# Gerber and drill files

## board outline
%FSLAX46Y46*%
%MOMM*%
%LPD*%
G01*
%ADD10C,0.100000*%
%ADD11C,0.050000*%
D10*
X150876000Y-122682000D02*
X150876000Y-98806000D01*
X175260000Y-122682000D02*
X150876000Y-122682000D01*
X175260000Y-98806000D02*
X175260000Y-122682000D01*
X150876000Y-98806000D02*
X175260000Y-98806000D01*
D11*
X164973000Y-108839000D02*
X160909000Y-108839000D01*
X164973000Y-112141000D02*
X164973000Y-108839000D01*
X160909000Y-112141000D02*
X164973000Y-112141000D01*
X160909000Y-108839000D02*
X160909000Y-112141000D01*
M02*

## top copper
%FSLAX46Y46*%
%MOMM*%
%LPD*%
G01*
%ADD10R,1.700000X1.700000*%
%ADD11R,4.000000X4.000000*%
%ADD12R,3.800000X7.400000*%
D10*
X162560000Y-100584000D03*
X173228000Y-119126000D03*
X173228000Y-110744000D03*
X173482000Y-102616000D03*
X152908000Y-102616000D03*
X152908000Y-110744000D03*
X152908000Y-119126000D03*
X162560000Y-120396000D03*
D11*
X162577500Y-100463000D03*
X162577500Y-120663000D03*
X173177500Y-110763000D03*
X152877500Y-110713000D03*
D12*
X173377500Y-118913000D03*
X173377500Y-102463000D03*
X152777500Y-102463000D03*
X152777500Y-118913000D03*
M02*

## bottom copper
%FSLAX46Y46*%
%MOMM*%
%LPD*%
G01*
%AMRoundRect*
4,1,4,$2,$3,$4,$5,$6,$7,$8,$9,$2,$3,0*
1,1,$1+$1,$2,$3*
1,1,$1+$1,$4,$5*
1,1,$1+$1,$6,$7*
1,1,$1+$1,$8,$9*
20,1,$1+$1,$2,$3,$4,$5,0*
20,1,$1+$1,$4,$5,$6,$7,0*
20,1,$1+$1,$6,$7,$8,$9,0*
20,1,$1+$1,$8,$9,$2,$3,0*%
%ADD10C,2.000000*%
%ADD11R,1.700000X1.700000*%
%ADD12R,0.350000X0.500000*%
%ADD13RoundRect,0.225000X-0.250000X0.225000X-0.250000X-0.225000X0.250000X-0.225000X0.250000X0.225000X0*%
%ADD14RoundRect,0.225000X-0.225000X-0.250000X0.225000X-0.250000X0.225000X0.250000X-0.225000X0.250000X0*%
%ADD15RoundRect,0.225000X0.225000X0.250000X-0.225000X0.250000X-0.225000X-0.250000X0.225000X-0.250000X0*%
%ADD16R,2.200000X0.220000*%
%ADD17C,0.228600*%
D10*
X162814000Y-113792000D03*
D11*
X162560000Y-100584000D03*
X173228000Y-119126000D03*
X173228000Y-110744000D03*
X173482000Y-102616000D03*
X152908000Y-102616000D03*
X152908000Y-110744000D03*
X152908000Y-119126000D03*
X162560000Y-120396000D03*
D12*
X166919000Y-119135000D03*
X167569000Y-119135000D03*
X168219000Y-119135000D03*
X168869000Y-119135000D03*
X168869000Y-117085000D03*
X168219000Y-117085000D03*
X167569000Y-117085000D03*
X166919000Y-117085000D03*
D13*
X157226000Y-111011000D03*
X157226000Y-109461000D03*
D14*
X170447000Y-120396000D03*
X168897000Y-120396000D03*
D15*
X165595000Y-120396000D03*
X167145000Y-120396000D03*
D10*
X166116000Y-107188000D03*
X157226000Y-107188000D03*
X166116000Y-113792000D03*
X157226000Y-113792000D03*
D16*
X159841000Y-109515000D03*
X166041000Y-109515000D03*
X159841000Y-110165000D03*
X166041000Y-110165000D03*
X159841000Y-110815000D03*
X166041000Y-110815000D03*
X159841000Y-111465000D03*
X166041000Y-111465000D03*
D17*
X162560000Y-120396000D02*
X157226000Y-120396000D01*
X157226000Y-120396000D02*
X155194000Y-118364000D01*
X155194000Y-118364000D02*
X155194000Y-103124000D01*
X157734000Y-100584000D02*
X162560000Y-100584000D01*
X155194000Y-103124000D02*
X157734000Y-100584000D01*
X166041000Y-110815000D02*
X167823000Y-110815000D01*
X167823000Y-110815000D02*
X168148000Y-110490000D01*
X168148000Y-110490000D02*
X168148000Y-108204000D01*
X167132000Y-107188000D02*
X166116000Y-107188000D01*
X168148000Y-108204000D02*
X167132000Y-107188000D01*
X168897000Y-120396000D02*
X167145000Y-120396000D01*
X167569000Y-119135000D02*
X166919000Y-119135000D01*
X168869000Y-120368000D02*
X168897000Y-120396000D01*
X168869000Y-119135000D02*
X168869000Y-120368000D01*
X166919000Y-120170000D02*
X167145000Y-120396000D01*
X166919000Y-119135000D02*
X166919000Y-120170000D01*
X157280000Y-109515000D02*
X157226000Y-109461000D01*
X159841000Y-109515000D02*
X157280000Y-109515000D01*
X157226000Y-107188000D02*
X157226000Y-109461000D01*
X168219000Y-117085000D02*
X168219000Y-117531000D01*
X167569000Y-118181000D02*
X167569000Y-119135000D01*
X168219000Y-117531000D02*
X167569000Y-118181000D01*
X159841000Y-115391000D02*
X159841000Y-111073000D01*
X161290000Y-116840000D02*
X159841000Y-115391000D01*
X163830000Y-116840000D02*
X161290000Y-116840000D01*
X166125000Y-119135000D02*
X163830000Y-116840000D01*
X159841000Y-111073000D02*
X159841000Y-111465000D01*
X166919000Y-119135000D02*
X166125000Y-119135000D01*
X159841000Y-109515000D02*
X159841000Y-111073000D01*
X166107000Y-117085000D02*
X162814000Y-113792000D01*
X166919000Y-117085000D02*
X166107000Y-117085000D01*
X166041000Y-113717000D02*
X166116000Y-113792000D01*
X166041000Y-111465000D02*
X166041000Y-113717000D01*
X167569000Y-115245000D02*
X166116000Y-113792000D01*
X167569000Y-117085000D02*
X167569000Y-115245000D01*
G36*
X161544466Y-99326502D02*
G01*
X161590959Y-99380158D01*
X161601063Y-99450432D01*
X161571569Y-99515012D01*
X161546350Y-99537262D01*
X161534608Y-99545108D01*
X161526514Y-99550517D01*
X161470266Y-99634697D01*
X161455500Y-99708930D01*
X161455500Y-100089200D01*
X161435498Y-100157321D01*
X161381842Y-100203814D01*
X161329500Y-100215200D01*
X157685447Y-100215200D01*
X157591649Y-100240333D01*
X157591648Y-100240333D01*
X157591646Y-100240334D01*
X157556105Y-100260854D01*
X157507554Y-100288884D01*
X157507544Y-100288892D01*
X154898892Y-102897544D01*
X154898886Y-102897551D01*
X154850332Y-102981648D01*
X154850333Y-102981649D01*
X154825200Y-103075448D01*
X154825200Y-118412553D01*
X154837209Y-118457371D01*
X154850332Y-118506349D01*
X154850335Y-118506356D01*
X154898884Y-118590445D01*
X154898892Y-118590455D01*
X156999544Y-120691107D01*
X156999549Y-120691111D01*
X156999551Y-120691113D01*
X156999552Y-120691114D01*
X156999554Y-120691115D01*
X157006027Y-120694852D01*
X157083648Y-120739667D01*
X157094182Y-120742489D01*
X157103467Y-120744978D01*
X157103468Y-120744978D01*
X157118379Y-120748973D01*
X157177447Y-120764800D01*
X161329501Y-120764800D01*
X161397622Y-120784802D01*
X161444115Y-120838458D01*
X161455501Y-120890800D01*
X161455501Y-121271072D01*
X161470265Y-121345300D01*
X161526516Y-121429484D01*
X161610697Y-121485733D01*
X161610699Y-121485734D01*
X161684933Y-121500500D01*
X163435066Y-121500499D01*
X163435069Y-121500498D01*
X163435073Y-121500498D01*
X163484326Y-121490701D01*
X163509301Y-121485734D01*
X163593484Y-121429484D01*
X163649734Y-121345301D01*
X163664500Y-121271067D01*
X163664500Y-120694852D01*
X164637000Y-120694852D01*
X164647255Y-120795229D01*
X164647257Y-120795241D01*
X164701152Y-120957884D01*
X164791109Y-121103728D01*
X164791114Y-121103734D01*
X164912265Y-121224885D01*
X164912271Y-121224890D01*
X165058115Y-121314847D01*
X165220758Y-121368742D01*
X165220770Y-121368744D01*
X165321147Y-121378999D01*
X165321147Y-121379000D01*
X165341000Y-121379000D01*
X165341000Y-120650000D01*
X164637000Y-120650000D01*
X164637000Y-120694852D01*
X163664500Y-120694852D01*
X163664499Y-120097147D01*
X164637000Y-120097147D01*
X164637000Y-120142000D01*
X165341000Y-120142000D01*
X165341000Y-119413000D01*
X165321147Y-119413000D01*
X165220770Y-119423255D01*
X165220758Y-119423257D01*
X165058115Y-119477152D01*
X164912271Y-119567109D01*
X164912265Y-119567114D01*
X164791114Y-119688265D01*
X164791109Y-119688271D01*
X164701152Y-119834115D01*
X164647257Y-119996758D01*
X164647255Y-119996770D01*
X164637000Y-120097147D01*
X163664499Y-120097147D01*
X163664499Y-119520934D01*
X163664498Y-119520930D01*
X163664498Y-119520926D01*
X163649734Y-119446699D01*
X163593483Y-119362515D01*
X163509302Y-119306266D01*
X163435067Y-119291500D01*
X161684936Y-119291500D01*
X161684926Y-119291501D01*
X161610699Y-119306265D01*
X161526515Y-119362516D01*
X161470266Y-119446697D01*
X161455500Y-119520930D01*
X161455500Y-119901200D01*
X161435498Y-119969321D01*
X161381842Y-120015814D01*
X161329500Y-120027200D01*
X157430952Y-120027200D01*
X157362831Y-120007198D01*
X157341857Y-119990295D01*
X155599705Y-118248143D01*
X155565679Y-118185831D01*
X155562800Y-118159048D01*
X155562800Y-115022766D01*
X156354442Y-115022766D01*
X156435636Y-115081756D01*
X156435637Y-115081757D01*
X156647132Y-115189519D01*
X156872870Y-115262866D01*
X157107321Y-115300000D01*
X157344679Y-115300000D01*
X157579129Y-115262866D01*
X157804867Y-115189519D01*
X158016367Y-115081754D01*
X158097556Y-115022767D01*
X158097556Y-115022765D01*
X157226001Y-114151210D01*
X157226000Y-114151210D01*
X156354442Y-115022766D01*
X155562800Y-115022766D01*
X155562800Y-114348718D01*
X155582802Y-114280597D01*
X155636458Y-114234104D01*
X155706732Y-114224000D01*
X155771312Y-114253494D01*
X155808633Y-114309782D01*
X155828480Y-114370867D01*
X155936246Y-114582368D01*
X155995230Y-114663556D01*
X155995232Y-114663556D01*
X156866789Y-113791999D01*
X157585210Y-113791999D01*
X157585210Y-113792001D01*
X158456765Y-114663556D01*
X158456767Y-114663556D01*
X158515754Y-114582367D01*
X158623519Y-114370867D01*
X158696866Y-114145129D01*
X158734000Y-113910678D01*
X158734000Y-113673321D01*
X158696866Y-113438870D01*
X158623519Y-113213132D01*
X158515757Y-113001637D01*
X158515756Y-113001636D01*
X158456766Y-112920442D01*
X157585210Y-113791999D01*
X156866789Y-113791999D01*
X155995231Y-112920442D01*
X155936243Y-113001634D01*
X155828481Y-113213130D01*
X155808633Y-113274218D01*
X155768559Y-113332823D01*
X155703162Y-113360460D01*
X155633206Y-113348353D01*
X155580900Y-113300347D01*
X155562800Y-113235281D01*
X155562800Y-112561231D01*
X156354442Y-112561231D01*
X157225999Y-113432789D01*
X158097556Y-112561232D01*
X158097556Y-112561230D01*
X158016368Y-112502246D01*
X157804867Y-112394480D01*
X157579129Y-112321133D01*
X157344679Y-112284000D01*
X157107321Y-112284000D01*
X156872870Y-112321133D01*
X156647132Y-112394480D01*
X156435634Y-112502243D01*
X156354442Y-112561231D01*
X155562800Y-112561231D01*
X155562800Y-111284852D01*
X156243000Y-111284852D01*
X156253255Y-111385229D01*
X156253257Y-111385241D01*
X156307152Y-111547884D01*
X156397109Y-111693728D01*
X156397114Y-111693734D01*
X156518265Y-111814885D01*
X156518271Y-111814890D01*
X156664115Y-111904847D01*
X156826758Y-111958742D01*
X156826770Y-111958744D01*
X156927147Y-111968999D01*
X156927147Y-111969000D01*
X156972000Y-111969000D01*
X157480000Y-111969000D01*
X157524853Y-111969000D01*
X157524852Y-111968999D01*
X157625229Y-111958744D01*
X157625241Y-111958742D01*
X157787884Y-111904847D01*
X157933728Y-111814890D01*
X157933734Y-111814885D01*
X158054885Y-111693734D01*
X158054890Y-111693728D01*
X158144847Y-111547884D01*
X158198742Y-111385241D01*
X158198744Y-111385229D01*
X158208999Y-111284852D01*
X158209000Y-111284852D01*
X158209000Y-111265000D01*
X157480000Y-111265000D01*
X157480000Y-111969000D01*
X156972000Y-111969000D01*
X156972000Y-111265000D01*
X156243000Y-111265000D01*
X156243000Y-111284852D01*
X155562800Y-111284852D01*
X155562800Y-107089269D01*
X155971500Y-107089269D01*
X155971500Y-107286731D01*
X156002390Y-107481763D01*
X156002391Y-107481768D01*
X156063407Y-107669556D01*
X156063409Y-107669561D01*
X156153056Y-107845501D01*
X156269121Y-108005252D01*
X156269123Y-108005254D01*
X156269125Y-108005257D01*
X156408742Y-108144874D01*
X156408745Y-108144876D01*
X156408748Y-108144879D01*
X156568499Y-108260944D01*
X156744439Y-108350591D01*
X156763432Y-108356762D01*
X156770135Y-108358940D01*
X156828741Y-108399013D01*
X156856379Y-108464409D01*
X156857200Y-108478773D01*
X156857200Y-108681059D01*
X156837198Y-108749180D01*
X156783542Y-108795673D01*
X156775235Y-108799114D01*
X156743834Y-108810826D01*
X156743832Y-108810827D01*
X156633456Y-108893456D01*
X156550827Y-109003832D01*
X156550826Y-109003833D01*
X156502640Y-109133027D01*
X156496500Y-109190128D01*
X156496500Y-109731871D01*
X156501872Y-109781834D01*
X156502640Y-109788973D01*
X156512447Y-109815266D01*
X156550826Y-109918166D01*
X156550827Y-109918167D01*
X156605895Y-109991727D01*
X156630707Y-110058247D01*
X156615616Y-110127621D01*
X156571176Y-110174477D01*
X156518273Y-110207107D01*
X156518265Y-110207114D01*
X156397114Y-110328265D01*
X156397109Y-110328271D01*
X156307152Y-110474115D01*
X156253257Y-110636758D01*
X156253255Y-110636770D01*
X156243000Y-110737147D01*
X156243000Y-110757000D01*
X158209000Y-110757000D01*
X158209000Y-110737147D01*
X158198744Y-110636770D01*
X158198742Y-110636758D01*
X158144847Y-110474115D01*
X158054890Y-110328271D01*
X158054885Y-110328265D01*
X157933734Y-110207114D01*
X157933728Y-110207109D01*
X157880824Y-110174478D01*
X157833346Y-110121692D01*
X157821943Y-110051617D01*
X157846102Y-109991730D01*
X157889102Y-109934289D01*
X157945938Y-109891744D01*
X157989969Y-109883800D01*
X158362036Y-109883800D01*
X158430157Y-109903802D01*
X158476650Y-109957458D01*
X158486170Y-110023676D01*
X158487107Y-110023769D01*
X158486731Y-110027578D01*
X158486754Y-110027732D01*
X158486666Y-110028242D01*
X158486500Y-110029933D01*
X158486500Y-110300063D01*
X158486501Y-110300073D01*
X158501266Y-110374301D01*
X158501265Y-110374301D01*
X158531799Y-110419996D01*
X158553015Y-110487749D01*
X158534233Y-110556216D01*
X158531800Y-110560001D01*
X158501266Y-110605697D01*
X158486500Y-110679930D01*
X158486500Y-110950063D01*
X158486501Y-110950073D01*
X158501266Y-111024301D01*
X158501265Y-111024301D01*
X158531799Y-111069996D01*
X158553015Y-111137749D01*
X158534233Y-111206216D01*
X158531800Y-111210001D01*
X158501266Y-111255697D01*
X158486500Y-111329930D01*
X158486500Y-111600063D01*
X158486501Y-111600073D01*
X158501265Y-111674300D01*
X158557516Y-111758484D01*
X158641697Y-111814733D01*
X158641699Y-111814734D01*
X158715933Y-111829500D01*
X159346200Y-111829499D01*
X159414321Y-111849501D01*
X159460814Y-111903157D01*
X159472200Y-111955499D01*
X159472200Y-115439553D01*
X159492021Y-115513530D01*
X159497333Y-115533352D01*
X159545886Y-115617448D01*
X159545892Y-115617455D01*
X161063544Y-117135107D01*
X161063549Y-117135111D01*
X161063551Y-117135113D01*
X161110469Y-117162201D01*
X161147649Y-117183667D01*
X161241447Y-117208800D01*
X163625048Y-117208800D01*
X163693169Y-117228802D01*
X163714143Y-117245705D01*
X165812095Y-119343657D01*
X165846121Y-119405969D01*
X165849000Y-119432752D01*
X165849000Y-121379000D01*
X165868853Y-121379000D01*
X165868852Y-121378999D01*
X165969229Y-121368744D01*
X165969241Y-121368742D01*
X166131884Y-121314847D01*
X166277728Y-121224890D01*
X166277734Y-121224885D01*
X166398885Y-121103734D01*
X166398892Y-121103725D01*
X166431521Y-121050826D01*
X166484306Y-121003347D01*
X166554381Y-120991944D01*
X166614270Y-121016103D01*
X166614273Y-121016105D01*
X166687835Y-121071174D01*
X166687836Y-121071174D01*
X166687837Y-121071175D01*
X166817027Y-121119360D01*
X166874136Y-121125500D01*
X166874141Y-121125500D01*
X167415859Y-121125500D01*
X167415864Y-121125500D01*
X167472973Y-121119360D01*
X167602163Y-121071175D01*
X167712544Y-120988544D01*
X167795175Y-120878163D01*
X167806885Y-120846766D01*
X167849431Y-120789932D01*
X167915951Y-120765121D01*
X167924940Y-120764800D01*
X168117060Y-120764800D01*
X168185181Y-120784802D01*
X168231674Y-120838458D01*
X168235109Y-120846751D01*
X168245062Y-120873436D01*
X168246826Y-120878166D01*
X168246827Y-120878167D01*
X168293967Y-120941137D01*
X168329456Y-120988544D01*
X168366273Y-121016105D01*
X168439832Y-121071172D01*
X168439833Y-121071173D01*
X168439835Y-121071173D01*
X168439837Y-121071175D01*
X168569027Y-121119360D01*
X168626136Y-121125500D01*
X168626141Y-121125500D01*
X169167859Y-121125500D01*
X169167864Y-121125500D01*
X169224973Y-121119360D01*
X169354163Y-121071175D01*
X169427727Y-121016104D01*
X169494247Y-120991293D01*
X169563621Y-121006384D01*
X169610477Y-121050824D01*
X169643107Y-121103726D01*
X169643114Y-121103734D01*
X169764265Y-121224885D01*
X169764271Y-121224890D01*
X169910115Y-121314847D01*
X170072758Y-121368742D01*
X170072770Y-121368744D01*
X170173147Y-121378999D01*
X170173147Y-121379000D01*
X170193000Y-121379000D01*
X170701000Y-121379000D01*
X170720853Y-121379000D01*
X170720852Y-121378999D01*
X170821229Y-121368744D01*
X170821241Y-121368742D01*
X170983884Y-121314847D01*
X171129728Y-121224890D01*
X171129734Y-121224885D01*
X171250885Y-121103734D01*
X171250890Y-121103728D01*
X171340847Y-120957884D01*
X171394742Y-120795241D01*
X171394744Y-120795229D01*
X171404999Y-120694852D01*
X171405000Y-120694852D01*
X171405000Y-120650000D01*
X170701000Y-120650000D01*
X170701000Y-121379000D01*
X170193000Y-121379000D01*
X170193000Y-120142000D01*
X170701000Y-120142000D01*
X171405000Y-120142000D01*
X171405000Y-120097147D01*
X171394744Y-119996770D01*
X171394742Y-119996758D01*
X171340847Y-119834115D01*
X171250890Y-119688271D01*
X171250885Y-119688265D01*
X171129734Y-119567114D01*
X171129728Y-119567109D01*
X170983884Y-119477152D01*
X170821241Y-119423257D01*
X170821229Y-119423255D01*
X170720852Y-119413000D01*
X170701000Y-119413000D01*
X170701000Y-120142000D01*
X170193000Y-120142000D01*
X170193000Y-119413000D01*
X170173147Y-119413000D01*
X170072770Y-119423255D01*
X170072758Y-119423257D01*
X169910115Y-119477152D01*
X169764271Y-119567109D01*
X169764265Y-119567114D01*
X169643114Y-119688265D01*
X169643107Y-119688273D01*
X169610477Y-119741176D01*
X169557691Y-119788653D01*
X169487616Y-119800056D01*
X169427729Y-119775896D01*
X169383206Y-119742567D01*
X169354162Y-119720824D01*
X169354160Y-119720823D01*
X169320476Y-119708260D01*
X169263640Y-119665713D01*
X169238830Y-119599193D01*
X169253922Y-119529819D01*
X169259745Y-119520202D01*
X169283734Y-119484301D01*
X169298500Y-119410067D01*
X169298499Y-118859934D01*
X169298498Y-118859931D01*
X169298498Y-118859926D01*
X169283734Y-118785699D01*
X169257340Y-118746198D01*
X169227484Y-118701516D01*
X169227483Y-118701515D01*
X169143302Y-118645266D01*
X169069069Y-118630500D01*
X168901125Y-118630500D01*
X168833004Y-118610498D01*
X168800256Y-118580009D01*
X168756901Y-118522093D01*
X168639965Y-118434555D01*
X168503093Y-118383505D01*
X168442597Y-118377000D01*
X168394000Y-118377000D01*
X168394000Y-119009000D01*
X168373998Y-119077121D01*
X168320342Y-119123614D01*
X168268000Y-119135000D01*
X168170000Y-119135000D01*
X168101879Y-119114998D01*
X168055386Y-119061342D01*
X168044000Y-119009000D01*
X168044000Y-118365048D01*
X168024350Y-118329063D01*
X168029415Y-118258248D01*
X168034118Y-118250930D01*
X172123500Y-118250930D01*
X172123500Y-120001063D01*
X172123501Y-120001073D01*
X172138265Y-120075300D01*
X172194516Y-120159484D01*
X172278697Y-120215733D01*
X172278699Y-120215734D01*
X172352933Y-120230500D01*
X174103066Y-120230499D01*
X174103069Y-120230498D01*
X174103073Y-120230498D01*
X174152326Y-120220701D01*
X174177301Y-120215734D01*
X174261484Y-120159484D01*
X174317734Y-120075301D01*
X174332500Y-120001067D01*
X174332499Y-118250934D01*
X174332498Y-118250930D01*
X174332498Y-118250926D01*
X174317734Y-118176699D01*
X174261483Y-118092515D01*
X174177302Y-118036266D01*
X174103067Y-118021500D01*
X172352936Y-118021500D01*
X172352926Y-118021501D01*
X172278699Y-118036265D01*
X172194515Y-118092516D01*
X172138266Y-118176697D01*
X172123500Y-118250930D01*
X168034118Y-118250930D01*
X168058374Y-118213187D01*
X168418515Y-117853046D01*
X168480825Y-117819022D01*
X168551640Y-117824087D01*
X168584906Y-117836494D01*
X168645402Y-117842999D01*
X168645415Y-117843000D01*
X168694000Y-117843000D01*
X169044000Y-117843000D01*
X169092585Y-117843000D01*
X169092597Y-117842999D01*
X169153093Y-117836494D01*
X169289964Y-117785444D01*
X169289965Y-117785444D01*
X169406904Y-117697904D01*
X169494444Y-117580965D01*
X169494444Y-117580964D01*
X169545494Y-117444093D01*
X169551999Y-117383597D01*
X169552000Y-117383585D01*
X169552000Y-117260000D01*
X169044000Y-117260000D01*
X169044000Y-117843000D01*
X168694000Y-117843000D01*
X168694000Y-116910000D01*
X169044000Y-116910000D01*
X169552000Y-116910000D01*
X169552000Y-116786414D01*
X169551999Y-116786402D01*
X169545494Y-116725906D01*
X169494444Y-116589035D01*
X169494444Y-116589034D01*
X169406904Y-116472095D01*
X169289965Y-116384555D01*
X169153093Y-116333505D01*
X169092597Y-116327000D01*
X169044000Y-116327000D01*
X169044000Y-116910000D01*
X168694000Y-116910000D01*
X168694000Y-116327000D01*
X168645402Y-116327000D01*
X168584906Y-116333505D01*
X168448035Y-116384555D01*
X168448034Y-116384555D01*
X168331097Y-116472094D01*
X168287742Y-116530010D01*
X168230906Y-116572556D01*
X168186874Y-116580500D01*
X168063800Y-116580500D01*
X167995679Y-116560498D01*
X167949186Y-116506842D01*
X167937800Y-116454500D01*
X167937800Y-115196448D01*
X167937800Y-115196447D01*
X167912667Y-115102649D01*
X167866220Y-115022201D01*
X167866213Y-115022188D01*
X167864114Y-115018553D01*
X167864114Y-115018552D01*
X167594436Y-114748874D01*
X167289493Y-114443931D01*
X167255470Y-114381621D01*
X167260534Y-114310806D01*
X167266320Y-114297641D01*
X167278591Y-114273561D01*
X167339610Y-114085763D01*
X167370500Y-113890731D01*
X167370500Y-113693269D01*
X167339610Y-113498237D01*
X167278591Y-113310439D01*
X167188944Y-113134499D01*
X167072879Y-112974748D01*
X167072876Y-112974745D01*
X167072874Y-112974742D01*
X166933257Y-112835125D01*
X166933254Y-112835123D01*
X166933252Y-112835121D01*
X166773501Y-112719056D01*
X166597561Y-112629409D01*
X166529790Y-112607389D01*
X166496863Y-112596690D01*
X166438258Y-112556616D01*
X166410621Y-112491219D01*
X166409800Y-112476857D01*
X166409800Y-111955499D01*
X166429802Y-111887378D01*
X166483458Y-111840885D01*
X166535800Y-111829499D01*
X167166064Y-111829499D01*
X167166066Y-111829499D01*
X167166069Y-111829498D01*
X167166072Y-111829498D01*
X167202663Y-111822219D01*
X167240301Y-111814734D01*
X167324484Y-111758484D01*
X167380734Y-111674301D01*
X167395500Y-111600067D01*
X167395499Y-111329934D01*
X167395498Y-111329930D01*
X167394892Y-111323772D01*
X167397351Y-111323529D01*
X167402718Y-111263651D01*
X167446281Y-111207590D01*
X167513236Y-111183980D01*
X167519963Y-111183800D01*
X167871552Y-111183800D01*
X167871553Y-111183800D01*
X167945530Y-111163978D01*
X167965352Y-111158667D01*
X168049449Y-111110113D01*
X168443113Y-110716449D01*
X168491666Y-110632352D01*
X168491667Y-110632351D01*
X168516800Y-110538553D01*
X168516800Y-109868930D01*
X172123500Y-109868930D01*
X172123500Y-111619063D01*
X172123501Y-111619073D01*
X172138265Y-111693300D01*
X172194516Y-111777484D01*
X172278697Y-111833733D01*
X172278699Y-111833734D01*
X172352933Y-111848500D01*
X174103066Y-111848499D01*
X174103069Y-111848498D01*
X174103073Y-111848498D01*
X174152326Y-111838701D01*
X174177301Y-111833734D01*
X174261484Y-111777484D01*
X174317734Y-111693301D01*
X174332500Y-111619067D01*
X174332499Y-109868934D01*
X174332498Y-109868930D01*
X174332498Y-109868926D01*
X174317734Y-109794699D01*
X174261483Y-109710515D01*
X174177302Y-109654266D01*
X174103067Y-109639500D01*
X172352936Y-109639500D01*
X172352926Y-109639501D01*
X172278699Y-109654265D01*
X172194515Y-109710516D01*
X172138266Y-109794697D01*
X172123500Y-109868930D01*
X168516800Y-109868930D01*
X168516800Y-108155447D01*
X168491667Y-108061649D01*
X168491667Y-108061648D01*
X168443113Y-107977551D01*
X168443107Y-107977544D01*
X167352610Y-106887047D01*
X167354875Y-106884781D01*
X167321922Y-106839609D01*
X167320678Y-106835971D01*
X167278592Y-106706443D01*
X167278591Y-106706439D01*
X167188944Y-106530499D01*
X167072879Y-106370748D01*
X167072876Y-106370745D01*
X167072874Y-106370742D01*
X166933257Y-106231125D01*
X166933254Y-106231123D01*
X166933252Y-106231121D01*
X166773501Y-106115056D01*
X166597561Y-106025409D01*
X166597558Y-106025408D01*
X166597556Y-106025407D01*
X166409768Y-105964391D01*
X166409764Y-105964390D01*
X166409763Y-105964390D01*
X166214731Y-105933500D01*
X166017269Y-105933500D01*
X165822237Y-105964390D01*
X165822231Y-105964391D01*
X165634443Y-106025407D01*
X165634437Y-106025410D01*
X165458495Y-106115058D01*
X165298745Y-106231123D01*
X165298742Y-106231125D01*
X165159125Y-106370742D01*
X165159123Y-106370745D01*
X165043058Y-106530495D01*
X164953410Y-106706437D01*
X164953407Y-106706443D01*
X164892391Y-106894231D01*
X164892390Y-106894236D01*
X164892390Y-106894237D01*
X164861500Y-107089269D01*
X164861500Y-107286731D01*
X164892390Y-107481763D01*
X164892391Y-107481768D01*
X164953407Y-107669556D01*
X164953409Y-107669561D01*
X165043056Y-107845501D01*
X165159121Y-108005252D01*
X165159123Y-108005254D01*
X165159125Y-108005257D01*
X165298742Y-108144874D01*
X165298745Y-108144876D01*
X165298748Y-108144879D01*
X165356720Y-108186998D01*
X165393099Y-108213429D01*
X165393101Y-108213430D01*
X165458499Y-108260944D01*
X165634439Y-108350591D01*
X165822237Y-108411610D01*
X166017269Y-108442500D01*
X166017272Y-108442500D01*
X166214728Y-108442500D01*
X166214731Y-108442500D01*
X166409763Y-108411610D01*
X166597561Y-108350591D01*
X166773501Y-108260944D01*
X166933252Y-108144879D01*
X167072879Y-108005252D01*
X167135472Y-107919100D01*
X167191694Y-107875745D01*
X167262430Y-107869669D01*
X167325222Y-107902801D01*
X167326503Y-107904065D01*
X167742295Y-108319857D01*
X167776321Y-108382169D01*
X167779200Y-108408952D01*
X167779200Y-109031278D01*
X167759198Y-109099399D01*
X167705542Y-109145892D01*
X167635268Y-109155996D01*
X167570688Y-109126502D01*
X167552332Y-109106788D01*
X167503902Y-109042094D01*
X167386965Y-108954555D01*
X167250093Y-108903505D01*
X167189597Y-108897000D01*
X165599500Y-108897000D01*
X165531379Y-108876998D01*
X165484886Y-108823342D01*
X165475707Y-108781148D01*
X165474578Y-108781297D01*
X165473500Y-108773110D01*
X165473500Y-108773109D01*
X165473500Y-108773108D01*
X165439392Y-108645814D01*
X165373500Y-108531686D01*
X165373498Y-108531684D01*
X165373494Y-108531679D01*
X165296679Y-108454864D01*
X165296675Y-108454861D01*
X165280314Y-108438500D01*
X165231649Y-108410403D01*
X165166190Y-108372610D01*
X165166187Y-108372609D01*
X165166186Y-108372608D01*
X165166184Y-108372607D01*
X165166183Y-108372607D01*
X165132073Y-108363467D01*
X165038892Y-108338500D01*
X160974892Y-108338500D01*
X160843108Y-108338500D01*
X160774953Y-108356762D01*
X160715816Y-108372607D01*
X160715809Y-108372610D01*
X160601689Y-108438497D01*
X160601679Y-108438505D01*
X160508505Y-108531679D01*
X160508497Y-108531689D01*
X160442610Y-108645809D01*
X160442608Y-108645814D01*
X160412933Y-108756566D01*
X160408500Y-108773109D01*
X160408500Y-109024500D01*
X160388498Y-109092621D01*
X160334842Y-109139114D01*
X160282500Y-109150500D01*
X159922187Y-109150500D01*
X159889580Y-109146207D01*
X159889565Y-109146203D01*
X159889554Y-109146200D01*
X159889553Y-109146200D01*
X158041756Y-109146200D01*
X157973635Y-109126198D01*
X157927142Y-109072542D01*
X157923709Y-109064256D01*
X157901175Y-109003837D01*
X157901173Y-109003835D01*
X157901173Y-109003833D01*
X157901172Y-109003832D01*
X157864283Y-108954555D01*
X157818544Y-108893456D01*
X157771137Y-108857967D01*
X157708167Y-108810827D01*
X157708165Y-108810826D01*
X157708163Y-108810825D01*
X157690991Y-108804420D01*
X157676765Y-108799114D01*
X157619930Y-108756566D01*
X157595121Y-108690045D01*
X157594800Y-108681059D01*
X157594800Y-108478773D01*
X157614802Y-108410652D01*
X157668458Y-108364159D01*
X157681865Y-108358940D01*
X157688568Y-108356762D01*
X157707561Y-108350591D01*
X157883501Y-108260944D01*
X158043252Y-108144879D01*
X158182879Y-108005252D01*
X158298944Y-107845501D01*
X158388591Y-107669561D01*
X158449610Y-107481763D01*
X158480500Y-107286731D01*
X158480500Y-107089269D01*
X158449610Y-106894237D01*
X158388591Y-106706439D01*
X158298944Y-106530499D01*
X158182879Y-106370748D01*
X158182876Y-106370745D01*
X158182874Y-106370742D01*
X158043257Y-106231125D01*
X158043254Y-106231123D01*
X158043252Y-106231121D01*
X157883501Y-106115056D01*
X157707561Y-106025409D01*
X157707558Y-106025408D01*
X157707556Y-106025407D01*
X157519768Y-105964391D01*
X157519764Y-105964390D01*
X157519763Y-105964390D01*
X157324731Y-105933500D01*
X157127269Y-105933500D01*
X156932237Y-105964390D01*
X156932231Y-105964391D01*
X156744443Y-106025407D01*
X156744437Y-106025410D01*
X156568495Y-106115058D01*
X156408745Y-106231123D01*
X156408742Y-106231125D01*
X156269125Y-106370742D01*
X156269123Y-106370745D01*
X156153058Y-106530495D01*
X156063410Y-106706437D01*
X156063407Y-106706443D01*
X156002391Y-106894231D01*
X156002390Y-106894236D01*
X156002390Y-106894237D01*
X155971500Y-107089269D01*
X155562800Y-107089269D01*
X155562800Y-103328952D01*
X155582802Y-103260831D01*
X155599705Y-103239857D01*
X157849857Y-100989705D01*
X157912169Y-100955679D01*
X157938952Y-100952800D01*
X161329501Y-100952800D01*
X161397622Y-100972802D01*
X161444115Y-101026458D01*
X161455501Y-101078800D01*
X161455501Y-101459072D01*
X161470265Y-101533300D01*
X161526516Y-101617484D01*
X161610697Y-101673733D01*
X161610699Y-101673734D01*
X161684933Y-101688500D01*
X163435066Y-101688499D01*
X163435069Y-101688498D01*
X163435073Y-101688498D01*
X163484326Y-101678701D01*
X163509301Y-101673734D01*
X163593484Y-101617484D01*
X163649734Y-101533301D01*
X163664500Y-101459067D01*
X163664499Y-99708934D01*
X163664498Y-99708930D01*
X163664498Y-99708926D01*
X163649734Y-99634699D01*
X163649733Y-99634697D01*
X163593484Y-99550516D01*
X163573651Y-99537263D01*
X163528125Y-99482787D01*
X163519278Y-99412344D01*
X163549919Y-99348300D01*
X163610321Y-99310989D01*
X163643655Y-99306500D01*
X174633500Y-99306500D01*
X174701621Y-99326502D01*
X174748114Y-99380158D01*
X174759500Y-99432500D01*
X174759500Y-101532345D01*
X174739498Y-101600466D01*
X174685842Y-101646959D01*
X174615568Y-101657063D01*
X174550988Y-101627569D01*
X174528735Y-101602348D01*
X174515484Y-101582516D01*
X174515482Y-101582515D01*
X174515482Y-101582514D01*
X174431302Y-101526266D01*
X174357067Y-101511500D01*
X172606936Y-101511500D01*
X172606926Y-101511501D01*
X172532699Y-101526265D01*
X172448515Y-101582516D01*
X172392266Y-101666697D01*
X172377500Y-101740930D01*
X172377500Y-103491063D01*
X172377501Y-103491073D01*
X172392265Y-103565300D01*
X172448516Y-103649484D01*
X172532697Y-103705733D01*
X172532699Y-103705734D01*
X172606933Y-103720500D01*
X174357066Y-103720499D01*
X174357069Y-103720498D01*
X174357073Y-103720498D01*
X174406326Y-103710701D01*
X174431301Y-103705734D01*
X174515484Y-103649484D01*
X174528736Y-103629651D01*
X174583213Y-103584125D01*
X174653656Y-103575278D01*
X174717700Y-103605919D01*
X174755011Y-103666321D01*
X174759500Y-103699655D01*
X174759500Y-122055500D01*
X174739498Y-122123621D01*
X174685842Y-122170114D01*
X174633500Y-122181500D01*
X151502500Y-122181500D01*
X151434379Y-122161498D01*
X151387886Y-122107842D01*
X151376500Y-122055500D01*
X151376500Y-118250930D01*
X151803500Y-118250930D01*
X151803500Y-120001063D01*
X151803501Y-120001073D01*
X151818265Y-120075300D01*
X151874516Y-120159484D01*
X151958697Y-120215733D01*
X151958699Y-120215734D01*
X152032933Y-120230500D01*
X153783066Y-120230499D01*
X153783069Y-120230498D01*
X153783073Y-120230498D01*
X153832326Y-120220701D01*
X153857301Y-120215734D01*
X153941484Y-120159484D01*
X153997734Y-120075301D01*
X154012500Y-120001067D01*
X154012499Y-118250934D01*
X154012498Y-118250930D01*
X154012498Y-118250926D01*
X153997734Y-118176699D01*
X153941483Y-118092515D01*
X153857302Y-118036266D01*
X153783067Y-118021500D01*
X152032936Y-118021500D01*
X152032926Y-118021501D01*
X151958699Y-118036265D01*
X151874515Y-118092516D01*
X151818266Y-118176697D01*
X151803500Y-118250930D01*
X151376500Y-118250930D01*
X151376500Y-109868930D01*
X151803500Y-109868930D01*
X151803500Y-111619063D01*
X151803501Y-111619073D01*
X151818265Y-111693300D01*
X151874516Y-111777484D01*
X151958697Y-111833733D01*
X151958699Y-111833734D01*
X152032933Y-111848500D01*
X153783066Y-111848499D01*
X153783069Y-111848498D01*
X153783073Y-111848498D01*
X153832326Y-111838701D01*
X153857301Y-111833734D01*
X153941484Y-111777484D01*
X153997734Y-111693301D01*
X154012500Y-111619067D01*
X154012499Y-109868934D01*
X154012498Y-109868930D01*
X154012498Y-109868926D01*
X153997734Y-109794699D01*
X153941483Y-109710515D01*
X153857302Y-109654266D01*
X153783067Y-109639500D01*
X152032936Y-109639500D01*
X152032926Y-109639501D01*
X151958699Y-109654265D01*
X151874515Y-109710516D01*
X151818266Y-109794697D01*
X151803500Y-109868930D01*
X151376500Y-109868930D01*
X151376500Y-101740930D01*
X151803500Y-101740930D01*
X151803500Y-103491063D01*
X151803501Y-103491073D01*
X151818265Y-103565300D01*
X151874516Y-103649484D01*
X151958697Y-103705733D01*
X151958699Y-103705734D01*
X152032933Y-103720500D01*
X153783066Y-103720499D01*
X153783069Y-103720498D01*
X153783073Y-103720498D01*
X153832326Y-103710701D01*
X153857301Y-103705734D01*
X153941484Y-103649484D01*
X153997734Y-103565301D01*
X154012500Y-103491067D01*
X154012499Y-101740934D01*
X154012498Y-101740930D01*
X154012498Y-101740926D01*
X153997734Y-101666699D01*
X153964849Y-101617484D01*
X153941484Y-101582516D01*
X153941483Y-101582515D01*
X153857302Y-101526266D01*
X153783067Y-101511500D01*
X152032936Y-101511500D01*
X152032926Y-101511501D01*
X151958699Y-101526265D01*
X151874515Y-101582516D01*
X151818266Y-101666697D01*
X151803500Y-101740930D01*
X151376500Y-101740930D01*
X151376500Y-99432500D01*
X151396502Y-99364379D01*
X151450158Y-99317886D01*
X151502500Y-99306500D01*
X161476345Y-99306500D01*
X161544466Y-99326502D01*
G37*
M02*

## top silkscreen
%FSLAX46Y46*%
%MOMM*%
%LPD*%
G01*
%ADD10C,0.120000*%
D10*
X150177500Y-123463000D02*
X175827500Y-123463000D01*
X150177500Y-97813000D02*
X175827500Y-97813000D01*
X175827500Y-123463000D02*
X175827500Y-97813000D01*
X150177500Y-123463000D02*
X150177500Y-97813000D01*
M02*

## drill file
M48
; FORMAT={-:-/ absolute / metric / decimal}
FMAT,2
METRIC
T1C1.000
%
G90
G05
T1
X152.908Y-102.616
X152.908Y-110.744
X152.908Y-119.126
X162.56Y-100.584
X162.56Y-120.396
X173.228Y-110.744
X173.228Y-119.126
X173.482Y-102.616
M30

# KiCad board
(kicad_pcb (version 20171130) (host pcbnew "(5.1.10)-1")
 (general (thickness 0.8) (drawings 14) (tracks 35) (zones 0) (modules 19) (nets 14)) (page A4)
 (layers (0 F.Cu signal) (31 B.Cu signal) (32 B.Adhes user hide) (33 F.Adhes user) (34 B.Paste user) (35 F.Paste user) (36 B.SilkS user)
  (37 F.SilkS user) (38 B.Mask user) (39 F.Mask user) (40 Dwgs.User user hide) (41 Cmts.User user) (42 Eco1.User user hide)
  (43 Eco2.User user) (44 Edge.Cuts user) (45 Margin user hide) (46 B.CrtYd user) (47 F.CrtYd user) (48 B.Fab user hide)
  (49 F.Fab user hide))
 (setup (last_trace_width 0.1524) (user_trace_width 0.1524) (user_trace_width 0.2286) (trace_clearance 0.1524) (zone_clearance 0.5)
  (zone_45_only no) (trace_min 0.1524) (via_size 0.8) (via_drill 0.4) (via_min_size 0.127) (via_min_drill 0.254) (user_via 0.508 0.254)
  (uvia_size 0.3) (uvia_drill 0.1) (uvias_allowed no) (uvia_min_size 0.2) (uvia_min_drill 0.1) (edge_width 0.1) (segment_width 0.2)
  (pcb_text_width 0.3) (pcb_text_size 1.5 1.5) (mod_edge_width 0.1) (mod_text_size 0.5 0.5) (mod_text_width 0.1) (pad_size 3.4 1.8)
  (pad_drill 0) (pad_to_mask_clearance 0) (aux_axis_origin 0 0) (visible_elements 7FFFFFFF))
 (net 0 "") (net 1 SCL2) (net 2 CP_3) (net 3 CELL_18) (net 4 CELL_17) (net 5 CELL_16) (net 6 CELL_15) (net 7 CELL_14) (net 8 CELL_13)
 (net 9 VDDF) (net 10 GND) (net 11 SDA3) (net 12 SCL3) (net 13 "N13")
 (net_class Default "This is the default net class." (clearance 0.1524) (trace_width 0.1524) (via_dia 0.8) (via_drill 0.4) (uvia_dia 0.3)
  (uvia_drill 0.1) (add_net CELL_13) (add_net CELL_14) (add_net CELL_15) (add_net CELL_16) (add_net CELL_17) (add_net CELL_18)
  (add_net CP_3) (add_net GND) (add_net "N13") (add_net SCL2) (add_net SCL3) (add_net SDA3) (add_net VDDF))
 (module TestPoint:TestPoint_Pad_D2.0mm (layer B.Cu) (at 162.814 113.792)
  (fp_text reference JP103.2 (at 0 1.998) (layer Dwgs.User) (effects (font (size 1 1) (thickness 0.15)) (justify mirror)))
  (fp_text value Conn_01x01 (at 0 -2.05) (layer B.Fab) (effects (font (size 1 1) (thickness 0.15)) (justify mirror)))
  (pad 1 smd circle (at 0 0) (size 2 2) (layers B.Cu B.Mask) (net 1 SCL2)))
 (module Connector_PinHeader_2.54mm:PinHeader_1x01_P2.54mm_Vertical (layer B.Cu) (at 162.56 100.584 270)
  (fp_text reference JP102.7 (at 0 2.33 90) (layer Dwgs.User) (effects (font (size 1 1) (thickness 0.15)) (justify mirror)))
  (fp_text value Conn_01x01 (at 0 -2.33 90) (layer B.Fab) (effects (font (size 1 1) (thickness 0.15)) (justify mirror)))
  (pad 1 thru_hole rect (at 0 0 270) (size 1.7 1.7) (drill 1) (layers *.Cu *.Mask) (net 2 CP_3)))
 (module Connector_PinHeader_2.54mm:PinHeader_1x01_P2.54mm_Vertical (layer B.Cu) (at 173.228 119.126 90)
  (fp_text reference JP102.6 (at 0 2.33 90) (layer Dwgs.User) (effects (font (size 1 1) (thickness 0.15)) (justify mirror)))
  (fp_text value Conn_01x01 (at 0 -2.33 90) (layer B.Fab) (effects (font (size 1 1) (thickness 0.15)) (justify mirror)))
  (pad 1 thru_hole rect (at 0 0 90) (size 1.7 1.7) (drill 1) (layers *.Cu *.Mask) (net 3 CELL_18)))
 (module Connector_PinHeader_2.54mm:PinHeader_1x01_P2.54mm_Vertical (layer B.Cu) (at 173.228 110.744 270)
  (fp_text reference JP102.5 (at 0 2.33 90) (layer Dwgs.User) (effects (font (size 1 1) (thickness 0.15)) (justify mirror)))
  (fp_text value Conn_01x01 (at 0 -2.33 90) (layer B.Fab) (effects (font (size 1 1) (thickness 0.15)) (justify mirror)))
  (pad 1 thru_hole rect (at 0 0 270) (size 1.7 1.7) (drill 1) (layers *.Cu *.Mask) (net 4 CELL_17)))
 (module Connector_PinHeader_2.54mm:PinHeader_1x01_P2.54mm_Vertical (layer B.Cu) (at 173.482 102.616 270)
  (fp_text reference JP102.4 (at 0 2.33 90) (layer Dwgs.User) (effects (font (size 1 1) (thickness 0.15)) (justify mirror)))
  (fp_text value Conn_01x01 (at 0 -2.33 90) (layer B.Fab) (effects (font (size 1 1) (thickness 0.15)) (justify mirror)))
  (pad 1 thru_hole rect (at 0 0 270) (size 1.7 1.7) (drill 1) (layers *.Cu *.Mask) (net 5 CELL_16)))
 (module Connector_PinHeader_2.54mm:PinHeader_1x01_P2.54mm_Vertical (layer B.Cu) (at 152.908 102.616 270)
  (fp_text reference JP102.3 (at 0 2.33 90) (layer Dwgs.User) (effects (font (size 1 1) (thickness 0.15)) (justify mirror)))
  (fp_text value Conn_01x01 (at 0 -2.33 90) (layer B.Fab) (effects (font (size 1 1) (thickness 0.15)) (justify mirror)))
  (pad 1 thru_hole rect (at 0 0 270) (size 1.7 1.7) (drill 1) (layers *.Cu *.Mask) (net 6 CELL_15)))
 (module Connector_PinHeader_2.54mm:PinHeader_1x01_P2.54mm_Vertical (layer B.Cu) (at 152.908 110.744 270)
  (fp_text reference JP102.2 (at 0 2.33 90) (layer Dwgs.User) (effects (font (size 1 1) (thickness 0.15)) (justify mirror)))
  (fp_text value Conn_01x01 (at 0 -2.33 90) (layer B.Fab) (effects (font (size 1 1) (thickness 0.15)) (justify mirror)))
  (pad 1 thru_hole rect (at 0 0 270) (size 1.7 1.7) (drill 1) (layers *.Cu *.Mask) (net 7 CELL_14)))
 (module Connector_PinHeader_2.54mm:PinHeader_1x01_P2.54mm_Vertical (layer B.Cu) (at 152.908 119.126 270)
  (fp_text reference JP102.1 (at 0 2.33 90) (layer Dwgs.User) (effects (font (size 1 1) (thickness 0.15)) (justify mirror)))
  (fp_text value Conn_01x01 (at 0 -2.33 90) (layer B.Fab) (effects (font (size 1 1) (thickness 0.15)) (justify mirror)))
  (pad 1 thru_hole rect (at 0 0 270) (size 1.7 1.7) (drill 1) (layers *.Cu *.Mask) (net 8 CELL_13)))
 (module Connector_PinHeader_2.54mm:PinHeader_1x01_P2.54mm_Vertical (layer B.Cu) (at 162.56 120.396)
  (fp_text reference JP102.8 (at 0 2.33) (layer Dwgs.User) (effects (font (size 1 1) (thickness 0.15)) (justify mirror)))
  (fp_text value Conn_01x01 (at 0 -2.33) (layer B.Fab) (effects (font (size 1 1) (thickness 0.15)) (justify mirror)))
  (pad 1 thru_hole rect (at 0 0) (size 1.7 1.7) (drill 1) (layers *.Cu *.Mask) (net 2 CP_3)))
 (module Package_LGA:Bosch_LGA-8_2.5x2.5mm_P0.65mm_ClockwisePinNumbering (layer B.Cu) (at 167.894 118.11 180)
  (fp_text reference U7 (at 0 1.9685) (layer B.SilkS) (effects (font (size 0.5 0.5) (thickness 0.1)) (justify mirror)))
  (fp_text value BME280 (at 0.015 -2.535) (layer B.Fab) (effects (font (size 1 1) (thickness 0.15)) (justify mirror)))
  (pad 5 smd rect (at 0.975 -1.025 90) (size 0.5 0.35) (layers B.Cu B.Paste B.Mask) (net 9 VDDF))
  (pad 6 smd rect (at 0.325 -1.025 90) (size 0.5 0.35) (layers B.Cu B.Paste B.Mask) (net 9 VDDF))
  (pad 7 smd rect (at -0.325 -1.025 90) (size 0.5 0.35) (layers B.Cu B.Paste B.Mask) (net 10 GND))
  (pad 8 smd rect (at -0.975 -1.025 90) (size 0.5 0.35) (layers B.Cu B.Paste B.Mask) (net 9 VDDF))
  (pad 1 smd rect (at -0.975 1.025 90) (size 0.5 0.35) (layers B.Cu B.Paste B.Mask) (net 10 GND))
  (pad 2 smd rect (at -0.325 1.025 90) (size 0.5 0.35) (layers B.Cu B.Paste B.Mask) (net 9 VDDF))
  (pad 3 smd rect (at 0.325 1.025 90) (size 0.5 0.35) (layers B.Cu B.Paste B.Mask) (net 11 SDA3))
  (pad 4 smd rect (at 0.975 1.025 90) (size 0.5 0.35) (layers B.Cu B.Paste B.Mask) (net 1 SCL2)))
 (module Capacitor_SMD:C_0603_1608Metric (layer B.Cu) (at 157.226 110.236 270)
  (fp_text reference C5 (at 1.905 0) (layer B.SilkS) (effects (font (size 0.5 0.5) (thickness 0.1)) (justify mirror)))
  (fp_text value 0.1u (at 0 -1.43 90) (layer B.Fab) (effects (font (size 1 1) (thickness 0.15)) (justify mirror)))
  (pad 2 smd roundrect (at 0.775 0 270) (size 0.9 0.95) (layers B.Cu B.Paste B.Mask) (roundrect_rratio 0.25) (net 10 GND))
  (pad 1 smd roundrect (at -0.775 0 270) (size 0.9 0.95) (layers B.Cu B.Paste B.Mask) (roundrect_rratio 0.25) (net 9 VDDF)))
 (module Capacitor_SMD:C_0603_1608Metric (layer B.Cu) (at 169.672 120.396)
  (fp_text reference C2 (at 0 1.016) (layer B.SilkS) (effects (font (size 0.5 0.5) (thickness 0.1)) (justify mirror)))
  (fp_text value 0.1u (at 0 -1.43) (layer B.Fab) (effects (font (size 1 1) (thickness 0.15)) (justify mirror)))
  (pad 2 smd roundrect (at 0.775 0) (size 0.9 0.95) (layers B.Cu B.Paste B.Mask) (roundrect_rratio 0.25) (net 10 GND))
  (pad 1 smd roundrect (at -0.775 0) (size 0.9 0.95) (layers B.Cu B.Paste B.Mask) (roundrect_rratio 0.25) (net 9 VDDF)))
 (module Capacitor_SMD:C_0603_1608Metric (layer B.Cu) (at 166.37 120.396 180)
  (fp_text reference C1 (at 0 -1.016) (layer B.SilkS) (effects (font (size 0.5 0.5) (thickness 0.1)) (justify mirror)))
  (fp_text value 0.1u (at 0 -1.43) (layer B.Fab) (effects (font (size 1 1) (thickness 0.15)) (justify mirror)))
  (pad 2 smd roundrect (at 0.775 0 180) (size 0.9 0.95) (layers B.Cu B.Paste B.Mask) (roundrect_rratio 0.25) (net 10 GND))
  (pad 1 smd roundrect (at -0.775 0 180) (size 0.9 0.95) (layers B.Cu B.Paste B.Mask) (roundrect_rratio 0.25) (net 9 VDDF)))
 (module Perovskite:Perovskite (layer F.Cu) (at 150.1775 123.463 90)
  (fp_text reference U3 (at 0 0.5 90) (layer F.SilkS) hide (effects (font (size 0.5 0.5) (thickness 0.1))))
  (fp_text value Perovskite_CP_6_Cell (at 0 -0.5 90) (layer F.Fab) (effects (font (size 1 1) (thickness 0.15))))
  (fp_line (start 0 0) (end 0 25.65) (layer F.SilkS) (width 0.12))
  (fp_line (start 25.65 0) (end 25.65 25.65) (layer F.SilkS) (width 0.12))
  (fp_line (start 0 25.65) (end 25.65 25.65) (layer F.SilkS) (width 0.12))
  (fp_line (start 0 0) (end 25.65 0) (layer F.SilkS) (width 0.12))
  (pad 7 smd rect (at 23 12.4 90) (size 4 4) (layers F.Cu F.Paste F.Mask) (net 2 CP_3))
  (pad 7 smd rect (at 2.8 12.4 90) (size 4 4) (layers F.Cu F.Paste F.Mask) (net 2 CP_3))
  (pad 5 smd rect (at 12.7 23 90) (size 4 4) (layers F.Cu F.Paste F.Mask) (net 4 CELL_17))
  (pad 2 smd rect (at 12.75 2.7 90) (size 4 4) (layers F.Cu F.Paste F.Mask) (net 7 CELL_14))
  (pad 6 smd rect (at 4.55 23.2 90) (size 7.4 3.8) (layers F.Cu F.Paste F.Mask) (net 3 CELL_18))
  (pad 4 smd rect (at 21 23.2 90) (size 7.4 3.8) (layers F.Cu F.Paste F.Mask) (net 5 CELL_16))
  (pad 3 smd rect (at 21 2.6 90) (size 7.4 3.8) (layers F.Cu F.Paste F.Mask) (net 6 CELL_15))
  (pad 1 smd rect (at 4.55 2.6 90) (size 7.4 3.8) (layers F.Cu F.Paste F.Mask) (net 8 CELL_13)))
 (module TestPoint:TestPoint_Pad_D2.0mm (layer B.Cu) (at 166.116 107.188)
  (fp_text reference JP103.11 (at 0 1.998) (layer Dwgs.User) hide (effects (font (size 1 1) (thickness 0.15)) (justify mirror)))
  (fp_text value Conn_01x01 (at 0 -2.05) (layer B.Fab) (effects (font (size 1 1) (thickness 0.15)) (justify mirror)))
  (pad 1 smd circle (at 0 0) (size 2 2) (layers B.Cu B.Mask) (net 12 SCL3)))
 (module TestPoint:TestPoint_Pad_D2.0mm (layer B.Cu) (at 157.226 107.188)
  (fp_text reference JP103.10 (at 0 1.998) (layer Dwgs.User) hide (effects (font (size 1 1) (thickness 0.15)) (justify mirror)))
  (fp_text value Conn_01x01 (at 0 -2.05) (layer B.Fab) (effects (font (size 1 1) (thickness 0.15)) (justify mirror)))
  (pad 1 smd circle (at 0 0) (size 2 2) (layers B.Cu B.Mask) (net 9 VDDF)))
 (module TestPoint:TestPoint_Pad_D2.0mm (layer B.Cu) (at 166.116 113.792)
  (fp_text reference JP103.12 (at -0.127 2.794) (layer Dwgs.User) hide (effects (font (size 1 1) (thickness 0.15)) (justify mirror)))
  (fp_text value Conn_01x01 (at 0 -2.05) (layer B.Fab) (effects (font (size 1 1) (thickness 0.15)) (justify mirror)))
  (pad 1 smd circle (at 0 0) (size 2 2) (layers B.Cu B.Mask) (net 11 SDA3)))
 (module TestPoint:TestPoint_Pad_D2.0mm (layer B.Cu) (at 157.226 113.792 90)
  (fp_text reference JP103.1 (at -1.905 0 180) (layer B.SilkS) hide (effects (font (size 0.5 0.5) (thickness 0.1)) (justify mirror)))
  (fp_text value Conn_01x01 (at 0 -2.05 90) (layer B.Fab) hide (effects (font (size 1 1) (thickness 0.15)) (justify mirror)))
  (pad 1 smd circle (at 0 0 90) (size 2 2) (layers B.Cu B.Mask) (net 10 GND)))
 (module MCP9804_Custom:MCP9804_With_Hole (layer B.Cu) (at 162.941 110.49)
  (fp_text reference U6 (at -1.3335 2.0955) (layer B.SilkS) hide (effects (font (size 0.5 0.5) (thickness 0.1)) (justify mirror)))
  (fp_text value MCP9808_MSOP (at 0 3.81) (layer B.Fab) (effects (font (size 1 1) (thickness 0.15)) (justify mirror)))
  (pad 5 smd rect (at -3.1 -0.975 90) (size 0.22 2.2) (layers B.Cu B.Paste B.Mask) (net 9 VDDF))
  (pad 4 smd rect (at 3.1 -0.975 90) (size 0.22 2.2) (layers B.Cu B.Paste B.Mask) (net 10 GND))
  (pad 6 smd rect (at -3.1 -0.325 90) (size 0.22 2.2) (layers B.Cu B.Paste B.Mask) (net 9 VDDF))
  (pad 3 smd rect (at 3.1 -0.325 90) (size 0.22 2.2) (layers B.Cu B.Paste B.Mask) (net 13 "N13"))
  (pad 7 smd rect (at -3.1 0.325 90) (size 0.22 2.2) (layers B.Cu B.Paste B.Mask) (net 9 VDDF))
  (pad 2 smd rect (at 3.1 0.325 90) (size 0.22 2.2) (layers B.Cu B.Paste B.Mask) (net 12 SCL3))
  (pad 8 smd rect (at -3.1 0.975 90) (size 0.22 2.2) (layers B.Cu B.Paste B.Mask) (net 9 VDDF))
  (pad 1 smd rect (at 3.1 0.975 90) (size 0.22 2.2) (layers B.Cu B.Paste B.Mask) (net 11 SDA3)))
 (gr_line (start 150.876 122.682) (end 150.876 98.806) (layer Edge.Cuts) (width 0.1))
 (gr_line (start 175.26 122.682) (end 150.876 122.682) (layer Edge.Cuts) (width 0.1))
 (gr_line (start 175.26 98.806) (end 175.26 122.682) (layer Edge.Cuts) (width 0.1))
 (gr_line (start 150.876 98.806) (end 175.26 98.806) (layer Edge.Cuts) (width 0.1))
 (gr_line (start 164.973 108.839) (end 160.909 108.839) (layer Edge.Cuts) (width 0.05))
 (gr_line (start 164.973 112.141) (end 164.973 108.839) (layer Edge.Cuts) (width 0.05))
 (gr_line (start 160.909 112.141) (end 164.973 112.141) (layer Edge.Cuts) (width 0.05))
 (gr_line (start 160.909 108.839) (end 160.909 112.141) (layer Edge.Cuts) (width 0.05))
 (segment (start 162.56 120.396) (end 157.226 120.396) (width 0.2286) (layer B.Cu) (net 2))
 (segment (start 157.226 120.396) (end 155.194 118.364) (width 0.2286) (layer B.Cu) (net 2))
 (segment (start 155.194 118.364) (end 155.194 103.124) (width 0.2286) (layer B.Cu) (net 2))
 (segment (start 157.734 100.584) (end 162.56 100.584) (width 0.2286) (layer B.Cu) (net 2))
 (segment (start 155.194 103.124) (end 157.734 100.584) (width 0.2286) (layer B.Cu) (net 2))
 (segment (start 166.041 110.815) (end 167.823 110.815) (width 0.2286) (layer B.Cu) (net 12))
 (segment (start 167.823 110.815) (end 168.148 110.49) (width 0.2286) (layer B.Cu) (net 12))
 (segment (start 168.148 110.49) (end 168.148 108.204) (width 0.2286) (layer B.Cu) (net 12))
 (segment (start 167.132 107.188) (end 166.116 107.188) (width 0.2286) (layer B.Cu) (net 12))
 (segment (start 168.148 108.204) (end 167.132 107.188) (width 0.2286) (layer B.Cu) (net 12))
 (segment (start 168.897 120.396) (end 167.145 120.396) (width 0.2286) (layer B.Cu) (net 9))
 (segment (start 167.569 119.135) (end 166.919 119.135) (width 0.2286) (layer B.Cu) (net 9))
 (segment (start 168.869 120.368) (end 168.897 120.396) (width 0.2286) (layer B.Cu) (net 9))
 (segment (start 168.869 119.135) (end 168.869 120.368) (width 0.2286) (layer B.Cu) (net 9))
 (segment (start 166.919 120.17) (end 167.145 120.396) (width 0.2286) (layer B.Cu) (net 9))
 (segment (start 166.919 119.135) (end 166.919 120.17) (width 0.2286) (layer B.Cu) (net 9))
 (segment (start 157.28 109.515) (end 157.226 109.461) (width 0.2286) (layer B.Cu) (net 9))
 (segment (start 159.841 109.515) (end 157.28 109.515) (width 0.2286) (layer B.Cu) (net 9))
 (segment (start 157.226 107.188) (end 157.226 109.461) (width 0.2286) (layer B.Cu) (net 9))
 (segment (start 168.219 117.085) (end 168.219 117.531) (width 0.2286) (layer B.Cu) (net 9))
 (segment (start 167.569 118.181) (end 167.569 119.135) (width 0.2286) (layer B.Cu) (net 9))
 (segment (start 168.219 117.531) (end 167.569 118.181) (width 0.2286) (layer B.Cu) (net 9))
 (segment (start 159.841 115.391) (end 159.841 111.073) (width 0.2286) (layer B.Cu) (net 9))
 (segment (start 161.29 116.84) (end 159.841 115.391) (width 0.2286) (layer B.Cu) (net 9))
 (segment (start 163.83 116.84) (end 161.29 116.84) (width 0.2286) (layer B.Cu) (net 9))
 (segment (start 166.125 119.135) (end 163.83 116.84) (width 0.2286) (layer B.Cu) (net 9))
 (segment (start 159.841 111.073) (end 159.841 111.465) (width 0.2286) (layer B.Cu) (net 9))
 (segment (start 166.919 119.135) (end 166.125 119.135) (width 0.2286) (layer B.Cu) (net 9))
 (segment (start 159.841 109.515) (end 159.841 111.073) (width 0.2286) (layer B.Cu) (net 9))
 (segment (start 166.107 117.085) (end 162.814 113.792) (width 0.2286) (layer B.Cu) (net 1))
 (segment (start 166.919 117.085) (end 166.107 117.085) (width 0.2286) (layer B.Cu) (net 1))
 (segment (start 166.041 113.717) (end 166.116 113.792) (width 0.2286) (layer B.Cu) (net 11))
 (segment (start 166.041 111.465) (end 166.041 113.717) (width 0.2286) (layer B.Cu) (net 11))
 (segment (start 167.569 115.245) (end 166.116 113.792) (width 0.2286) (layer B.Cu) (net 11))
 (segment (start 167.569 117.085) (end 167.569 115.245) (width 0.2286) (layer B.Cu) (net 11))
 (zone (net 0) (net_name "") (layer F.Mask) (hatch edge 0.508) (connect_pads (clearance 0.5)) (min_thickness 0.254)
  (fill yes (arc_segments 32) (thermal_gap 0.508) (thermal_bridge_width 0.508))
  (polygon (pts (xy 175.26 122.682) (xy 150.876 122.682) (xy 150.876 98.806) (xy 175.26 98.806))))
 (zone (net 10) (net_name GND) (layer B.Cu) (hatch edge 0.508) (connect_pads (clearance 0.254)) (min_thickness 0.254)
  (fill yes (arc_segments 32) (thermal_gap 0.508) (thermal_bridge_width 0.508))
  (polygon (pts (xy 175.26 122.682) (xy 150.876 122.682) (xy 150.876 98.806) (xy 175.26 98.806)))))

